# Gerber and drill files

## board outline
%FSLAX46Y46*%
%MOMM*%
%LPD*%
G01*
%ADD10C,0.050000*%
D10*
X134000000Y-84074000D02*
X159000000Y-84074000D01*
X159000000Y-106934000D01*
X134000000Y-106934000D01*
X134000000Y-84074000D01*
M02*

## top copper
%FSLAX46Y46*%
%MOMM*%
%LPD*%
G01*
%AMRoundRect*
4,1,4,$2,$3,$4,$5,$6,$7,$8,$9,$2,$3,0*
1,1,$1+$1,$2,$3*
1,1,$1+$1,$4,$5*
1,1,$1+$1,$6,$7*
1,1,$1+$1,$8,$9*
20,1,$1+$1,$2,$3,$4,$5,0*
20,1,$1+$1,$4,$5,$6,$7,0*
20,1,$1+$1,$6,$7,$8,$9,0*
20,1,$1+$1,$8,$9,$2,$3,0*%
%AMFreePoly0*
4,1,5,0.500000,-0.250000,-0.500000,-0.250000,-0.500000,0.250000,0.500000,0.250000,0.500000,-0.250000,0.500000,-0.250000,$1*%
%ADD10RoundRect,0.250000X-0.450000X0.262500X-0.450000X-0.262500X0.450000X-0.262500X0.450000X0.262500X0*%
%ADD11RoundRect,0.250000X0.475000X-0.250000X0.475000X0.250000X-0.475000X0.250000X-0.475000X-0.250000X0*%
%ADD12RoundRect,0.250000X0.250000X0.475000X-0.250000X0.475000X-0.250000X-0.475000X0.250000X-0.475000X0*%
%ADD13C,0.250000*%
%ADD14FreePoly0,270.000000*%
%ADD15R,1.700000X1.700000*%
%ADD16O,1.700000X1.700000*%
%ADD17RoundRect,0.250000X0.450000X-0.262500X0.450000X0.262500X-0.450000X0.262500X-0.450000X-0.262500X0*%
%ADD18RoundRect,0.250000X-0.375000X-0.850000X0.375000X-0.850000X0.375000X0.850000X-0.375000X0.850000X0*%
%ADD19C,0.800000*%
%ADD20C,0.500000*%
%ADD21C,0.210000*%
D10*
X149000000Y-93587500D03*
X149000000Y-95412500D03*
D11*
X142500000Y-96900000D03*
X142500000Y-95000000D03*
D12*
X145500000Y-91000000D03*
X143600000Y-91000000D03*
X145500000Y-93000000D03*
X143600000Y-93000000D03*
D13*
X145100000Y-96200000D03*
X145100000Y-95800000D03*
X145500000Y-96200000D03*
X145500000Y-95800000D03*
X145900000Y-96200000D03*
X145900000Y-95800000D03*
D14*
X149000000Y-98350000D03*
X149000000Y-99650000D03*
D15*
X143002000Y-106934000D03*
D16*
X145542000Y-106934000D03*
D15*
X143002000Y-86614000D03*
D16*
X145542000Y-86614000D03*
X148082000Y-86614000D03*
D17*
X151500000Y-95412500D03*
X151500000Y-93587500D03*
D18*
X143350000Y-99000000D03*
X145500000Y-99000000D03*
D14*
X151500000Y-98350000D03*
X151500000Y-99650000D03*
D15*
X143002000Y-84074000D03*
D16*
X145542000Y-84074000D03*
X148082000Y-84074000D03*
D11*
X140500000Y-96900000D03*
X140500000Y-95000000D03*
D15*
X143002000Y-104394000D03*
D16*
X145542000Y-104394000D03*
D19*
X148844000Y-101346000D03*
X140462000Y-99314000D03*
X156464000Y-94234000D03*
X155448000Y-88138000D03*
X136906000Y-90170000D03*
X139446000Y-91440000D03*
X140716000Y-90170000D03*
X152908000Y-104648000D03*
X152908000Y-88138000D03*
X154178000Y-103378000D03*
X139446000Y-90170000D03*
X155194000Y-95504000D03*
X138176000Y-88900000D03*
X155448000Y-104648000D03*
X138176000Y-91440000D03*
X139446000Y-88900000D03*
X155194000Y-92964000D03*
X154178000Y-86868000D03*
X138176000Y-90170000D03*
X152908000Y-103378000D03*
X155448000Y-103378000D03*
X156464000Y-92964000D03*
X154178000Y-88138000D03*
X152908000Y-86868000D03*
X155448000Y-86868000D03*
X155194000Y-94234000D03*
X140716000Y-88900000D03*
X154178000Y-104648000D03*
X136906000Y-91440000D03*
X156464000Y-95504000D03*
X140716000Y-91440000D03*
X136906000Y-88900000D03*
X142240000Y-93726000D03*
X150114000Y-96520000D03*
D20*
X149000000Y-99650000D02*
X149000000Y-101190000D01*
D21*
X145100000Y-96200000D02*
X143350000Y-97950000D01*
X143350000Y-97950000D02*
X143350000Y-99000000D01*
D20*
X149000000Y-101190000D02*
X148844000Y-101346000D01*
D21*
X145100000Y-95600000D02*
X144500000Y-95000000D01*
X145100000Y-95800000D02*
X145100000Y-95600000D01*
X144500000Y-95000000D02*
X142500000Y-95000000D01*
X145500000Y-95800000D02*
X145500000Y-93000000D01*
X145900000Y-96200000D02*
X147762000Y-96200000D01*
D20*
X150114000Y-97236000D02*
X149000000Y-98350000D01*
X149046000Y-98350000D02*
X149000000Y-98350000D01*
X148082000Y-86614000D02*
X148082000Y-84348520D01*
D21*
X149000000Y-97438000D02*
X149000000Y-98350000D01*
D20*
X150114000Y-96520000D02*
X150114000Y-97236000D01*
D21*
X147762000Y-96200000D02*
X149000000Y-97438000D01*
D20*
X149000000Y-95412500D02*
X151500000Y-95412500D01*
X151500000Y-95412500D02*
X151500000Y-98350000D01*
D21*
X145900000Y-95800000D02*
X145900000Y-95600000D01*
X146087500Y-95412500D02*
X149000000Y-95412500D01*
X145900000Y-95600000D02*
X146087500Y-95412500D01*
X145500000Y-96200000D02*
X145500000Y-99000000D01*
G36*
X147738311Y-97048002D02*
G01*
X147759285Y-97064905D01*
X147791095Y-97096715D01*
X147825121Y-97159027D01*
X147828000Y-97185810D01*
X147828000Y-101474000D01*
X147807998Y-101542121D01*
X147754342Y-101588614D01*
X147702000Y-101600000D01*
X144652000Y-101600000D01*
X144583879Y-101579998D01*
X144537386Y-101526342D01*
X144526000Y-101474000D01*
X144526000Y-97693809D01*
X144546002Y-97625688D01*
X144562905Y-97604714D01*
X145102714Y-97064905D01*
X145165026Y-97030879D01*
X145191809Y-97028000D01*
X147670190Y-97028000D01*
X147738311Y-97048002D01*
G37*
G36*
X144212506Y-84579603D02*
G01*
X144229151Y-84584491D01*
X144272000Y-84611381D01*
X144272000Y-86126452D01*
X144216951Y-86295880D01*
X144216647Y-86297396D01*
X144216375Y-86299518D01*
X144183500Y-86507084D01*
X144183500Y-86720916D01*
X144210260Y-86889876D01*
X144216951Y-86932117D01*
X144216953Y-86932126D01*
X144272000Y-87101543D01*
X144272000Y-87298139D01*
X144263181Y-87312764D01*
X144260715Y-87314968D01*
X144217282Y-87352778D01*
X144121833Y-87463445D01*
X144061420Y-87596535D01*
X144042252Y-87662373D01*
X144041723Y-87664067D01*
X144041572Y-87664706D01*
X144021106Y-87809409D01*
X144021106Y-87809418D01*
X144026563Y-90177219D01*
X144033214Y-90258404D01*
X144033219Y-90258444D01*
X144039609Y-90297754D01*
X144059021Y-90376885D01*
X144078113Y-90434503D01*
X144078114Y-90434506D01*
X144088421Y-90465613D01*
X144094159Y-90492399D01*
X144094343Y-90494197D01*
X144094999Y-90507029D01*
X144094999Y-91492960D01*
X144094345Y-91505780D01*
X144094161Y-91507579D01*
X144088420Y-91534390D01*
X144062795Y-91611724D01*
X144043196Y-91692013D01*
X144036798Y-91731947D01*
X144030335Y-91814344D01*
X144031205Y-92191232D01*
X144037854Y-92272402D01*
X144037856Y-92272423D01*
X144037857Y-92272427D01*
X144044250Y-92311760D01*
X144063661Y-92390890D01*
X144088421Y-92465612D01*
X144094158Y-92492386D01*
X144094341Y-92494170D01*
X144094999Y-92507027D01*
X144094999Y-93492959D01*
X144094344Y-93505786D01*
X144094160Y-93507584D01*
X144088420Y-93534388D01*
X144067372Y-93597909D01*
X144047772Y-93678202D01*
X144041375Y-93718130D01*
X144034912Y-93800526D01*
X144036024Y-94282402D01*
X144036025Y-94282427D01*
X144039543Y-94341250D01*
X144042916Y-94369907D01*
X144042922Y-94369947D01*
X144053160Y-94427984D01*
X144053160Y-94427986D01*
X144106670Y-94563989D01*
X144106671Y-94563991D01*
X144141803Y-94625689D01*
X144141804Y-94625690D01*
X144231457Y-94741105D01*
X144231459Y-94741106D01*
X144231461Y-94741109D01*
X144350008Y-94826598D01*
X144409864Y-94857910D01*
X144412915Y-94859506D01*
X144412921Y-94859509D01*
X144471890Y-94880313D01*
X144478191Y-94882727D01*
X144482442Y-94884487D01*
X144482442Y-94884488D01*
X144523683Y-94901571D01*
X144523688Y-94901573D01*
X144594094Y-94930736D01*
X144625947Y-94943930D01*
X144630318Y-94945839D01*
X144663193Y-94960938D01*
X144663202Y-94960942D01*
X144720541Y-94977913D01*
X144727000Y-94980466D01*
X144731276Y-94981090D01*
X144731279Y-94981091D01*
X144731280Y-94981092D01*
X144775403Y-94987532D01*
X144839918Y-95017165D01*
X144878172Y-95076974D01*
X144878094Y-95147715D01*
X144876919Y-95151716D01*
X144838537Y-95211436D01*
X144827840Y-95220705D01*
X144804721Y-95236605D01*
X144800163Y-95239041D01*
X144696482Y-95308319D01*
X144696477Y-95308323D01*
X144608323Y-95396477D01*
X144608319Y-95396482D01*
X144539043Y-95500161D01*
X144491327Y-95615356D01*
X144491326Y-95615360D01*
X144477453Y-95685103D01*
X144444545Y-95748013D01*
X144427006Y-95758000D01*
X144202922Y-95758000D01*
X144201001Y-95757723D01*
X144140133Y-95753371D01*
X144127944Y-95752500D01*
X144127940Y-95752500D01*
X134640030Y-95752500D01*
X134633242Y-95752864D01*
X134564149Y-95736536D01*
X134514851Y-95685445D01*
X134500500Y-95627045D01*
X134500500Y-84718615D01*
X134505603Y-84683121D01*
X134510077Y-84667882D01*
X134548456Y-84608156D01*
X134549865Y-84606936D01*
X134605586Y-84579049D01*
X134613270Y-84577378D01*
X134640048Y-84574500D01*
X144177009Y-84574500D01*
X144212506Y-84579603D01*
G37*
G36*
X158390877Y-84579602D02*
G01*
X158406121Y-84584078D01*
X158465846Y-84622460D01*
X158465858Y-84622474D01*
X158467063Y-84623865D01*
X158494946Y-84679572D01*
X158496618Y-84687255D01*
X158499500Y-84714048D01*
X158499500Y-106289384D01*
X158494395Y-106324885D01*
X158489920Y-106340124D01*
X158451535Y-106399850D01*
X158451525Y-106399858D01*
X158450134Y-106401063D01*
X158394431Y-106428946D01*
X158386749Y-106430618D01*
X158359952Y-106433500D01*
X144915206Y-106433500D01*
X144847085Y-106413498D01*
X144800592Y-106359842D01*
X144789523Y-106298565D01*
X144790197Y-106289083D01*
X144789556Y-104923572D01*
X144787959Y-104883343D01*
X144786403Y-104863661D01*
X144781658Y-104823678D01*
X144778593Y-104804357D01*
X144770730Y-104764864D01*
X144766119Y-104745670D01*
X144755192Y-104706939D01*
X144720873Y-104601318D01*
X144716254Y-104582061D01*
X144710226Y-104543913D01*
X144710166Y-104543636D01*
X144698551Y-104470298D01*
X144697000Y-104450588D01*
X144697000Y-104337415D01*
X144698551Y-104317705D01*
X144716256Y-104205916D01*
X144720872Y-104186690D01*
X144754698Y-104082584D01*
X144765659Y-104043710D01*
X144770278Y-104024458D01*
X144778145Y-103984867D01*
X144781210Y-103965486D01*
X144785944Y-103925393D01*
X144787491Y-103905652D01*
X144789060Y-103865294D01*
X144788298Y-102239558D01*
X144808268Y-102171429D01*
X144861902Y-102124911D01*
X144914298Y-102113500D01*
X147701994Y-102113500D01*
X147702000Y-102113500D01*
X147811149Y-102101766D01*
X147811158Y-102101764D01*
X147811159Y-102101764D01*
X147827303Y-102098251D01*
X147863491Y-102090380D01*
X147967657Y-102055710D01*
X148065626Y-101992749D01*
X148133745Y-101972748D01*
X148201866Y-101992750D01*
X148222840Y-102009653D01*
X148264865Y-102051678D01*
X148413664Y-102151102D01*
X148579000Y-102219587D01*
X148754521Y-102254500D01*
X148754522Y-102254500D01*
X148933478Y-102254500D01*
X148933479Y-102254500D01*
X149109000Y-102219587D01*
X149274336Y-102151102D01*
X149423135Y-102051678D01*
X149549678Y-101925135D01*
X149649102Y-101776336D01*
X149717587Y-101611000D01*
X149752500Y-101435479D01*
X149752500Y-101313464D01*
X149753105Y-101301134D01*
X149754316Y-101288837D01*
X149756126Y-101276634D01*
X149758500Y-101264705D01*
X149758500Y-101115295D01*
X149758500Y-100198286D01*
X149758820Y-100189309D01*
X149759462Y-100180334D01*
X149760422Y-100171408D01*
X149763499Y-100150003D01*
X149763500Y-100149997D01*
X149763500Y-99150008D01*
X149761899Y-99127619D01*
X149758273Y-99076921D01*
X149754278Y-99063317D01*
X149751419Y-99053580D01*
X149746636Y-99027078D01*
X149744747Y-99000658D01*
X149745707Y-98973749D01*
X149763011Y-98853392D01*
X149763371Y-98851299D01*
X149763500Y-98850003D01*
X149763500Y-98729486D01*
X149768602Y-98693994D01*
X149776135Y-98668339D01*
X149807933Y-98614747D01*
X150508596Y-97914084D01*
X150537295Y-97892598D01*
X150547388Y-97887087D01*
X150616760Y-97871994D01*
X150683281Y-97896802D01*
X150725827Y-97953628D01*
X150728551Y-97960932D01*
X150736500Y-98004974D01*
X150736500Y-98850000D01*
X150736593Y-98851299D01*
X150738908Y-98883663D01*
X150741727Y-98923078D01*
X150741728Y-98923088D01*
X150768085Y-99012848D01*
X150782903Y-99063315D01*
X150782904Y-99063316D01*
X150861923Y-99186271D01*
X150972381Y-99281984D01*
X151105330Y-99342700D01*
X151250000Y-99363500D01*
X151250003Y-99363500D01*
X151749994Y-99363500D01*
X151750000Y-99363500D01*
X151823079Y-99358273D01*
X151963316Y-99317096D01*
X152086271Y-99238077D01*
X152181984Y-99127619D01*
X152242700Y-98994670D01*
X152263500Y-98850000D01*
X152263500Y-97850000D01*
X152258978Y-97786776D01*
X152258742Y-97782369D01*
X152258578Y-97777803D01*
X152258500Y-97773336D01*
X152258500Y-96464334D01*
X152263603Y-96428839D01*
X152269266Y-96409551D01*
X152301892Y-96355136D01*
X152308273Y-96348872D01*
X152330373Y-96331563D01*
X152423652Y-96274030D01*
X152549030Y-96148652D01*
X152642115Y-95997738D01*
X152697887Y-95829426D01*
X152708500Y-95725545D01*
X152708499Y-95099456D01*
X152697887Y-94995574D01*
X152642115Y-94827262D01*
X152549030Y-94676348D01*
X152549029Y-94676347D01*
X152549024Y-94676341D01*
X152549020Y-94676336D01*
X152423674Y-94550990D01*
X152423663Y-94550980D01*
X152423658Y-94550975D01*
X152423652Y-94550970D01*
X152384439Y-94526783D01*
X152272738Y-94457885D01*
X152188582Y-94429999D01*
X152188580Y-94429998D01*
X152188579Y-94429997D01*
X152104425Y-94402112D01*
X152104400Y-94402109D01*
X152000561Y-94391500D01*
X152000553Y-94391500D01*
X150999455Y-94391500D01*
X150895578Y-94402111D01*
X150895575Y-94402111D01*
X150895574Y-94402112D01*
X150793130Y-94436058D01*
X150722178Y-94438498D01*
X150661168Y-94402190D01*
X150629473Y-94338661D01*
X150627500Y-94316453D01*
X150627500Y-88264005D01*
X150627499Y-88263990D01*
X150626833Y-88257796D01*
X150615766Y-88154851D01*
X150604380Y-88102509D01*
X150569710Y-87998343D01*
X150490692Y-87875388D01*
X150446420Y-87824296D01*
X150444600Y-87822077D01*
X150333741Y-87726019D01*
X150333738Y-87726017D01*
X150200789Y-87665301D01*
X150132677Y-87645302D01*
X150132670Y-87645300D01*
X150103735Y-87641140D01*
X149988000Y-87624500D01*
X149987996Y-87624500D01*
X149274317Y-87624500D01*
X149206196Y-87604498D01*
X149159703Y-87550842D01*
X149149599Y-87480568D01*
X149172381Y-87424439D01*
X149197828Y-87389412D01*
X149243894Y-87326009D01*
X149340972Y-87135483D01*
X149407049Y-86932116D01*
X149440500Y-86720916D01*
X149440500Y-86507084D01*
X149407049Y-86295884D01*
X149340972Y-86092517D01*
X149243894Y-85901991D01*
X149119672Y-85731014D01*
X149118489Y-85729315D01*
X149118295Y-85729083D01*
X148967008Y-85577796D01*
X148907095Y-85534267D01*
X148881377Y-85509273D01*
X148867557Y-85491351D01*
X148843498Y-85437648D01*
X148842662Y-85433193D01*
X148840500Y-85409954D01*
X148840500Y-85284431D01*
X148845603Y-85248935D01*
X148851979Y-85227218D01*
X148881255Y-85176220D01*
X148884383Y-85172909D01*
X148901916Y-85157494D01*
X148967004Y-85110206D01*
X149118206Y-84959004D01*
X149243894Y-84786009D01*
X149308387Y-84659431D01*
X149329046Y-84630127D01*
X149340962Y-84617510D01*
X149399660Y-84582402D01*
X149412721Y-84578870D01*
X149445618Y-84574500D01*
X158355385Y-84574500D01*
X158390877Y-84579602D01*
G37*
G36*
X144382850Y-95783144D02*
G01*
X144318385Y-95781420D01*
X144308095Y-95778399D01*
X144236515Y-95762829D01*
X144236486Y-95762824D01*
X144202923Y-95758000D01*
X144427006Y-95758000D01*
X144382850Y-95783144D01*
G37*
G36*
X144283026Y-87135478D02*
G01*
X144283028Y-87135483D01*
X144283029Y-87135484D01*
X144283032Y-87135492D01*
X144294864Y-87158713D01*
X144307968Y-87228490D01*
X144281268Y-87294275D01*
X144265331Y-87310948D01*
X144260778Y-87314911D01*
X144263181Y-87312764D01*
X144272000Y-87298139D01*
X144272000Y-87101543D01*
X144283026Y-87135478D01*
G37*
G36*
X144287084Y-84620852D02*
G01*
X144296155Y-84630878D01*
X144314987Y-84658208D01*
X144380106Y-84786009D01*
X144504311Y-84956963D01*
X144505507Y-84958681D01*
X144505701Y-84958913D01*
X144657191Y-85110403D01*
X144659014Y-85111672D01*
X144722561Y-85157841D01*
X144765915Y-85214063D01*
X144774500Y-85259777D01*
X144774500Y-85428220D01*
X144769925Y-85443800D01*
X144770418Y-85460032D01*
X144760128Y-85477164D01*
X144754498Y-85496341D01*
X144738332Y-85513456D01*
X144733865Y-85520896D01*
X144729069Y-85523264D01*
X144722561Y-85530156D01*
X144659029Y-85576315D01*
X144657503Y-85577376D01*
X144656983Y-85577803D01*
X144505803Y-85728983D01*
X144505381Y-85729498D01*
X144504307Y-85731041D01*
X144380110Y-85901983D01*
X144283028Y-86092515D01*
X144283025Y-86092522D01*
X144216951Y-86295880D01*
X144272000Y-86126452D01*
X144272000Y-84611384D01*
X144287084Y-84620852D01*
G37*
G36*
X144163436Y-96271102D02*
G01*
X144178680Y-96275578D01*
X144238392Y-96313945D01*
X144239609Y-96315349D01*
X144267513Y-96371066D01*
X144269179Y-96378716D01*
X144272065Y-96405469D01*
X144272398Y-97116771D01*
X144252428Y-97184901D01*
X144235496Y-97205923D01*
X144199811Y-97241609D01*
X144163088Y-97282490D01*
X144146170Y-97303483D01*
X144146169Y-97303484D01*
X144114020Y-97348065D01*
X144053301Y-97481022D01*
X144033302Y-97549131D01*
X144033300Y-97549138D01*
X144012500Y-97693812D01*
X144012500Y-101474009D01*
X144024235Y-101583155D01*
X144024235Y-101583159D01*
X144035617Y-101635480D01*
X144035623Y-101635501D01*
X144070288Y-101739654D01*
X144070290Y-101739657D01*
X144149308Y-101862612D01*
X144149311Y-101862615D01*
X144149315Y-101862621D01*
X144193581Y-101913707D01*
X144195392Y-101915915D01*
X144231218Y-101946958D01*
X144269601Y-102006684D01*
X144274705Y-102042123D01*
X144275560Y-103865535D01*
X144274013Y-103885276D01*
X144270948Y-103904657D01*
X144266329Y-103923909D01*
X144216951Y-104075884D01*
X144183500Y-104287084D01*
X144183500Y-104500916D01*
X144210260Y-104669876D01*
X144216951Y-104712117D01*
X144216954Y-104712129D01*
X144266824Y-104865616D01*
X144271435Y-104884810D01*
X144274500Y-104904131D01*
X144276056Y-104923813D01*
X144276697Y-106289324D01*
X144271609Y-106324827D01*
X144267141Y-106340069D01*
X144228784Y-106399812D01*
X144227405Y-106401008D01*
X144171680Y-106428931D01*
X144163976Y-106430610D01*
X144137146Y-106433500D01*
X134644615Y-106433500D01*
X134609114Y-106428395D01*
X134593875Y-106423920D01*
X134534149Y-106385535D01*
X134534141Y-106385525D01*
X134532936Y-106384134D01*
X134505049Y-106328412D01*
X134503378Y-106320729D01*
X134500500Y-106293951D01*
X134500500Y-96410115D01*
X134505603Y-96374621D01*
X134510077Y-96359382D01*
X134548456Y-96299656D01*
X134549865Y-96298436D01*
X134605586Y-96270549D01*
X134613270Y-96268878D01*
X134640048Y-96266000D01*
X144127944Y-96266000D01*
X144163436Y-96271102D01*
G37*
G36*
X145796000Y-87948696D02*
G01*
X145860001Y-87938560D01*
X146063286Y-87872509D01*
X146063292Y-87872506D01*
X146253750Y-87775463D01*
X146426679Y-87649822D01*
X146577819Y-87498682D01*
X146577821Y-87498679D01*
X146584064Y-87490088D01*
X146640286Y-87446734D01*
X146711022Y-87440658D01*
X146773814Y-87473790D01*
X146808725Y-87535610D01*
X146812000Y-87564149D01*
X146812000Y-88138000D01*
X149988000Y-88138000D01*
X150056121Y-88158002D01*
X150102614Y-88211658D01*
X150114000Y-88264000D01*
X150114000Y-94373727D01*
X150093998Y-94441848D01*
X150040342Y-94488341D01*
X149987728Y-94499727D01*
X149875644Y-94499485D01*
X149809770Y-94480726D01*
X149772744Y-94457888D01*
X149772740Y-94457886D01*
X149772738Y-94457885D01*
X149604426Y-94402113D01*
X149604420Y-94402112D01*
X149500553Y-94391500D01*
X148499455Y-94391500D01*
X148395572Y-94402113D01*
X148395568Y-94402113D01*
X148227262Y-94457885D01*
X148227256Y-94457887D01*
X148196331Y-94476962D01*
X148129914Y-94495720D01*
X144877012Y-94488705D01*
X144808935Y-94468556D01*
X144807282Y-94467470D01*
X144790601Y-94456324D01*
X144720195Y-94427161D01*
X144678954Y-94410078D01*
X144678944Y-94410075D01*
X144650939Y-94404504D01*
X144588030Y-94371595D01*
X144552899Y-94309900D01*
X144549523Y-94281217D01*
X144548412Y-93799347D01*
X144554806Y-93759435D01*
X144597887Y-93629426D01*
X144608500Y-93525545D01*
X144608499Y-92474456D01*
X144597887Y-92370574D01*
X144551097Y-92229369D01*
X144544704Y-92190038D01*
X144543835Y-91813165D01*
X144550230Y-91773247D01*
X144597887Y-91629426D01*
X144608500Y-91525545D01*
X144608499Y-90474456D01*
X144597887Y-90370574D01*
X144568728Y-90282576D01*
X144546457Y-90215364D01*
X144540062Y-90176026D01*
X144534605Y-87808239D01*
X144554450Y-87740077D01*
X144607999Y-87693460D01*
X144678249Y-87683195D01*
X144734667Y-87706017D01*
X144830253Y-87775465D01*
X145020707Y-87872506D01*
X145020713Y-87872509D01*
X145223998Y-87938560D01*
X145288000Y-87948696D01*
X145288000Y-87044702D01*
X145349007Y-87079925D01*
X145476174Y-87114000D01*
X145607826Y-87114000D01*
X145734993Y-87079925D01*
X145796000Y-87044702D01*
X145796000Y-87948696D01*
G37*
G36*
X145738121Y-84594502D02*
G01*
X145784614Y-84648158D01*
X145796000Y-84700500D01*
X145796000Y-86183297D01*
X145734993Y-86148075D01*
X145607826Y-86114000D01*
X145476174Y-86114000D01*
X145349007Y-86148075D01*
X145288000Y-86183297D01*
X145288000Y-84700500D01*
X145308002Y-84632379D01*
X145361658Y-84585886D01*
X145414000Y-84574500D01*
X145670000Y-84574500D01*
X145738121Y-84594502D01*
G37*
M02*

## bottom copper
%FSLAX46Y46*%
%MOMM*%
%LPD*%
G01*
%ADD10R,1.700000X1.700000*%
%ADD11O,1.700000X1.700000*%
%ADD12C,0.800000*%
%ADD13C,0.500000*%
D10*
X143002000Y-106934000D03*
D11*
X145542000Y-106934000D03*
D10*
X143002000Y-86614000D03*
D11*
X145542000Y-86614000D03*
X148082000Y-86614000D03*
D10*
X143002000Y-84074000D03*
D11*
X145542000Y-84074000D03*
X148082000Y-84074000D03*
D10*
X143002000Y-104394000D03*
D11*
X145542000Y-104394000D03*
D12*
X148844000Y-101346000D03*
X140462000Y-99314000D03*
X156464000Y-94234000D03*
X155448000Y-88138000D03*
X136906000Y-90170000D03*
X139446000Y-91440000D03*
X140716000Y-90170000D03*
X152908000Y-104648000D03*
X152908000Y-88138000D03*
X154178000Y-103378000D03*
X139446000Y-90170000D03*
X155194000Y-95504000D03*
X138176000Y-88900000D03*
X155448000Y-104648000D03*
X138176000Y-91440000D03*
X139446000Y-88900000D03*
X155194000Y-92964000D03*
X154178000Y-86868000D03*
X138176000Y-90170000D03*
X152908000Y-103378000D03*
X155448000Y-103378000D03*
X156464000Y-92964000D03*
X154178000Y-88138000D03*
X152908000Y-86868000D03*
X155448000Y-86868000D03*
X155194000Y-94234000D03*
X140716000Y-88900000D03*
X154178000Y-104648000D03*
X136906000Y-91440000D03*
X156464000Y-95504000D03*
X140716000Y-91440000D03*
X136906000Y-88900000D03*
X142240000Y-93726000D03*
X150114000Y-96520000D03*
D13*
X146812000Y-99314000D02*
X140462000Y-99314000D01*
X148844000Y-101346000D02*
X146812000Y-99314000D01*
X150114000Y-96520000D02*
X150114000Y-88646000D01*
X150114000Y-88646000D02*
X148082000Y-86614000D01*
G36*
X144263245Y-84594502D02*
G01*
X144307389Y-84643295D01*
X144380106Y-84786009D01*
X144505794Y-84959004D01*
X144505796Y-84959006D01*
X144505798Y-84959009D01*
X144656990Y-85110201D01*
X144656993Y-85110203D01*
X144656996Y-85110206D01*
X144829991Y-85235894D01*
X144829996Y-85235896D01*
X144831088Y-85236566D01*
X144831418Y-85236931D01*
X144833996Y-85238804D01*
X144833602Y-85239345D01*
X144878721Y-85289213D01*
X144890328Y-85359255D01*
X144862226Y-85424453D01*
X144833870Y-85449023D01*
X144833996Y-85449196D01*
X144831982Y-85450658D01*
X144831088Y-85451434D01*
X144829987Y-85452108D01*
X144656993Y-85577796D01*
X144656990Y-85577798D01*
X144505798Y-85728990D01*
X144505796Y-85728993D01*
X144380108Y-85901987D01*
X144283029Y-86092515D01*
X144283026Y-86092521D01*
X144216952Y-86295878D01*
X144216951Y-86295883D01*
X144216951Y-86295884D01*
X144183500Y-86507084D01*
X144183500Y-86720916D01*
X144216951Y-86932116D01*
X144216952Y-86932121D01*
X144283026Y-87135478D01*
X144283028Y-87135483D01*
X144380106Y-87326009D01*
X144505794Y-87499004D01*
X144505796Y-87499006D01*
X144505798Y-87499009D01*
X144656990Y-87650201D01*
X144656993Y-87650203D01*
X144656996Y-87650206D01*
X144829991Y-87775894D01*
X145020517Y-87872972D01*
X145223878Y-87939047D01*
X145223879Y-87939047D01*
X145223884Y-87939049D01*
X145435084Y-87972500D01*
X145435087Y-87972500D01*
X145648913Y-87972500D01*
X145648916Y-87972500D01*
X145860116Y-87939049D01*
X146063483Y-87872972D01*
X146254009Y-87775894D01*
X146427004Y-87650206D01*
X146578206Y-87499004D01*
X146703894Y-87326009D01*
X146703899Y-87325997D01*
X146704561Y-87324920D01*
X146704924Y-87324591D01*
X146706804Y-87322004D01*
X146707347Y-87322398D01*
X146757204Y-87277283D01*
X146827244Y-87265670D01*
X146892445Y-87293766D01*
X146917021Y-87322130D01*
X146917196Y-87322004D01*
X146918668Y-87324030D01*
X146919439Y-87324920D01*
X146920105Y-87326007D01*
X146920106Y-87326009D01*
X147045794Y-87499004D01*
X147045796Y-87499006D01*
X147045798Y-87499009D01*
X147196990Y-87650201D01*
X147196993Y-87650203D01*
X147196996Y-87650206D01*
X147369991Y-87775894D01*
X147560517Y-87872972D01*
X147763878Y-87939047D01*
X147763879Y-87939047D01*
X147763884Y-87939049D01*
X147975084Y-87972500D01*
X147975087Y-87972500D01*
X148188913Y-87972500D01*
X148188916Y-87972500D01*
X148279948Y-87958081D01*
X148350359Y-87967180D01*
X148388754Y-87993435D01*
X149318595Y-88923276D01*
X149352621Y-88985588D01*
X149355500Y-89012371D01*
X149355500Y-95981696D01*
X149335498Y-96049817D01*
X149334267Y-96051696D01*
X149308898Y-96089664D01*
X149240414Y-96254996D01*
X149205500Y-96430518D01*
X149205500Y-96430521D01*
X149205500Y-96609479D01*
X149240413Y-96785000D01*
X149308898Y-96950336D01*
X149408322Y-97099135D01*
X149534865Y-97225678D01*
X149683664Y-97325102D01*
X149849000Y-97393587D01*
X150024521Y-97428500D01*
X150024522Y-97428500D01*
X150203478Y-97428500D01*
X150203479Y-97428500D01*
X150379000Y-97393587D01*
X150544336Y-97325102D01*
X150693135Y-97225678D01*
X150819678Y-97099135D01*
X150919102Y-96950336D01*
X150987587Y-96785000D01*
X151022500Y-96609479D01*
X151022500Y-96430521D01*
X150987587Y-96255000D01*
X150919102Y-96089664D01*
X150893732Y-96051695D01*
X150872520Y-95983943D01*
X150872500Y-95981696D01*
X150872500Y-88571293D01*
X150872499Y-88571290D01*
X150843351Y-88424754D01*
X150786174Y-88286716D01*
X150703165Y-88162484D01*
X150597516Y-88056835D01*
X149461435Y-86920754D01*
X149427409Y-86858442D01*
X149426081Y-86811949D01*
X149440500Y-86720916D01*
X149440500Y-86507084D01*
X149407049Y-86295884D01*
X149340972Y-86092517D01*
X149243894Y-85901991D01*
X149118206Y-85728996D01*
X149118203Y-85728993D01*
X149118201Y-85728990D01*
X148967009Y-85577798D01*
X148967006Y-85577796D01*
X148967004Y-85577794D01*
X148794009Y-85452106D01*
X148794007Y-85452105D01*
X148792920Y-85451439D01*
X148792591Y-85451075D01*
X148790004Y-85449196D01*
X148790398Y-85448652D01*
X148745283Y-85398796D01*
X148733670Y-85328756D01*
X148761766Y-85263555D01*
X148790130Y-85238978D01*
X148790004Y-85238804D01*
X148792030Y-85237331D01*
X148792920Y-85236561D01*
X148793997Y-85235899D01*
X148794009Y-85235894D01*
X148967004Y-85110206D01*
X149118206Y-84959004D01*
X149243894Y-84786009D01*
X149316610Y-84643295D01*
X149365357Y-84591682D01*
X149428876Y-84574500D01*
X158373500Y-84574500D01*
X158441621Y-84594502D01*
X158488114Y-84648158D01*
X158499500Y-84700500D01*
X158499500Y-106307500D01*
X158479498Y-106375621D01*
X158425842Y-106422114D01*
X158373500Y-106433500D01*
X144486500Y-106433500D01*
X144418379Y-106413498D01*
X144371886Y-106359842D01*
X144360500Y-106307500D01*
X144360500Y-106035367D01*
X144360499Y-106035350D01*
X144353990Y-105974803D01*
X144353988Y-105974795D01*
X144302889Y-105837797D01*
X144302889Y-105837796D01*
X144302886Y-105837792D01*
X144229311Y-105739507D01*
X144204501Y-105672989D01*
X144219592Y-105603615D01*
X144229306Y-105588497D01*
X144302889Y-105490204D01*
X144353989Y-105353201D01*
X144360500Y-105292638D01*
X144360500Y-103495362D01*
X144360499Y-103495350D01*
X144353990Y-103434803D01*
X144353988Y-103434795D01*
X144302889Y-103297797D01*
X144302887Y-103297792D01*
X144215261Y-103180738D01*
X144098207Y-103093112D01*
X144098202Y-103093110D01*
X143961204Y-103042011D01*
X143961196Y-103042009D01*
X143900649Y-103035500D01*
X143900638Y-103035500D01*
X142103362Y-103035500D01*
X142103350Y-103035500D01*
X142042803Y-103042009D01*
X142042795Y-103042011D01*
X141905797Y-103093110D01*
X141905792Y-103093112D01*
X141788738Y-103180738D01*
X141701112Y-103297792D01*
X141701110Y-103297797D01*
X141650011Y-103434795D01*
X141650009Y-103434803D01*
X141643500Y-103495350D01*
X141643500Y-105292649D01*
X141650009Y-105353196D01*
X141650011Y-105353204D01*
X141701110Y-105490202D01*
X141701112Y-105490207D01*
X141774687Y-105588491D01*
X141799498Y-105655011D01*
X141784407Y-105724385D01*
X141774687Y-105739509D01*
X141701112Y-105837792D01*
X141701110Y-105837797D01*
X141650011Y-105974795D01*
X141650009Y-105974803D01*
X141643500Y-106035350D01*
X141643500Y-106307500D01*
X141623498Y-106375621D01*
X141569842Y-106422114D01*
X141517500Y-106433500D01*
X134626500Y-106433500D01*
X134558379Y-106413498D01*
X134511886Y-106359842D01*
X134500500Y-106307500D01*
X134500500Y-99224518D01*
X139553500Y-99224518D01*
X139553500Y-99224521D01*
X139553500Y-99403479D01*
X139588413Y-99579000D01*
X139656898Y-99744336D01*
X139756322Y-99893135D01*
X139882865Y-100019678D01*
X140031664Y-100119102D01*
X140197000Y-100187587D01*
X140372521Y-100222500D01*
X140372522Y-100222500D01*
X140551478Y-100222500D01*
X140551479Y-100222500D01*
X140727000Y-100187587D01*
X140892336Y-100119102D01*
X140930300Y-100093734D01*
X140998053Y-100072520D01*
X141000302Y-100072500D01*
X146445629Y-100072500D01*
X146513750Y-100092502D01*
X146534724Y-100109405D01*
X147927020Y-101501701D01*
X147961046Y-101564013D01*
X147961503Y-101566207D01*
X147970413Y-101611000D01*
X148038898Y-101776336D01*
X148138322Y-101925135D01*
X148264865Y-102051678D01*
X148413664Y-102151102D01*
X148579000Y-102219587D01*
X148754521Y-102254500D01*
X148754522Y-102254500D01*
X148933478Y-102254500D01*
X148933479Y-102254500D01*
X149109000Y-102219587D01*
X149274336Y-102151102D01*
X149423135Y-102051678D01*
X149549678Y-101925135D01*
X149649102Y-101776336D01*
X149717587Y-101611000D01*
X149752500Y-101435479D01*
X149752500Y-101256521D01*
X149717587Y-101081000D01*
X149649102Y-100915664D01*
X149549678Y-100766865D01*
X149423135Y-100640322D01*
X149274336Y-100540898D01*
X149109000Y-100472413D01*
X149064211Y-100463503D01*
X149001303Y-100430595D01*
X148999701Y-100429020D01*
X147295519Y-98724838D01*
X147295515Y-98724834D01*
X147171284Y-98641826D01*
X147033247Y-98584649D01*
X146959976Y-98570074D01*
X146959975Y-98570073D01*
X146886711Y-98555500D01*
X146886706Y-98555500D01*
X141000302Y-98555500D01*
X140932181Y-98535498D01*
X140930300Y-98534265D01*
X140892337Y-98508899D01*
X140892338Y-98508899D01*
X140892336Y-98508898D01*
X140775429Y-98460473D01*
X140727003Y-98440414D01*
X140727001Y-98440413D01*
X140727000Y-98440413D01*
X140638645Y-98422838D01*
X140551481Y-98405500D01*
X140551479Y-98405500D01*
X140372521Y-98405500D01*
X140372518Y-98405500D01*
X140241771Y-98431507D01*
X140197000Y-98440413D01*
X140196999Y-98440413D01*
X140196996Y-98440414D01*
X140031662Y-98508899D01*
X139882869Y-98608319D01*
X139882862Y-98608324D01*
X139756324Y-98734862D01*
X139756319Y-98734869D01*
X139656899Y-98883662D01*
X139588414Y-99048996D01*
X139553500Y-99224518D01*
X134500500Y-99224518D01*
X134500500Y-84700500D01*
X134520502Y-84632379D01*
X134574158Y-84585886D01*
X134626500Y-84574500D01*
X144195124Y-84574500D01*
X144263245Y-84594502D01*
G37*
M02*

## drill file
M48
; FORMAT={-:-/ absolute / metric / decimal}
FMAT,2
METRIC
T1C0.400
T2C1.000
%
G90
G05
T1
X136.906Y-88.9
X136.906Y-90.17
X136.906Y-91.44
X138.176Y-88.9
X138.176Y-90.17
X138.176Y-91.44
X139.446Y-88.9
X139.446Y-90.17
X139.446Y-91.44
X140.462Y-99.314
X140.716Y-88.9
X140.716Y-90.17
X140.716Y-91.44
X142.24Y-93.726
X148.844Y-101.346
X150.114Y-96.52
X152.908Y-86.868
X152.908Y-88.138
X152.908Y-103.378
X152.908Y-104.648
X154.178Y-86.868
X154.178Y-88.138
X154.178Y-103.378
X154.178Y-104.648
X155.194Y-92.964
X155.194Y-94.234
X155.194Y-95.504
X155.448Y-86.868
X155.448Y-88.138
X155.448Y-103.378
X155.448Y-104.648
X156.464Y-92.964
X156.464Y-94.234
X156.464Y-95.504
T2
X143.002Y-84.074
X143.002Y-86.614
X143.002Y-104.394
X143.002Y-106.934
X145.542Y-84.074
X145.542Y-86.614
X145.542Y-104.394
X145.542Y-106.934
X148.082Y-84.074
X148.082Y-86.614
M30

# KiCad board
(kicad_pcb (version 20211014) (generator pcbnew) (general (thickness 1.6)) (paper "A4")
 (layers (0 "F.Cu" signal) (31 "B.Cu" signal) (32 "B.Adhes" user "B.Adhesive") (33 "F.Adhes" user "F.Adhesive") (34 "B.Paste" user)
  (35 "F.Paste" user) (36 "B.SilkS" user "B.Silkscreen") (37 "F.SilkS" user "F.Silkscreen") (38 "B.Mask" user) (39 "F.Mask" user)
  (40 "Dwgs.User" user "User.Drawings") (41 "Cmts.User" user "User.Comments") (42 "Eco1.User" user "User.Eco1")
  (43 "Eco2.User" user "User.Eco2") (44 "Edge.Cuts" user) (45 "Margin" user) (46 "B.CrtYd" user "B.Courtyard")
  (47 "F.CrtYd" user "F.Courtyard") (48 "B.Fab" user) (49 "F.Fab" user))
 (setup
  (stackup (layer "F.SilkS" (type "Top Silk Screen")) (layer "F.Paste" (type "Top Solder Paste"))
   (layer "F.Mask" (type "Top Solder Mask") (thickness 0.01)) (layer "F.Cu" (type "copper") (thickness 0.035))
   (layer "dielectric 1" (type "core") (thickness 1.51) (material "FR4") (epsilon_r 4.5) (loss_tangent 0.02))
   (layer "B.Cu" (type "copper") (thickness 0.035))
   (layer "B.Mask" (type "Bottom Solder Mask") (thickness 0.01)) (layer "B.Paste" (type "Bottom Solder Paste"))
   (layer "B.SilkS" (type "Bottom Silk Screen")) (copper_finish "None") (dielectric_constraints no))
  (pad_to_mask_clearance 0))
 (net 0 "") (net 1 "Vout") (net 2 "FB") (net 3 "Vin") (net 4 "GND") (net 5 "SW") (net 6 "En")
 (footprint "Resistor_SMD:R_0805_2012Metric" (layer "F.Cu") (at 149 94.5 -90) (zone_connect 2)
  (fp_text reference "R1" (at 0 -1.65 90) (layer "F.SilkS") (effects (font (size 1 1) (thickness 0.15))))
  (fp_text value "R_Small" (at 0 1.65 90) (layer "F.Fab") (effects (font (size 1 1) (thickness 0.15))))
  (pad "1" smd roundrect (at -0.9125 0 270) (size 1.025 1.4) (layers "F.Cu" "F.Paste" "F.Mask") (roundrect_rratio 0.243902) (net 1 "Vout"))
  (pad "2" smd roundrect (at 0.9125 0 270) (size 1.025 1.4) (layers "F.Cu" "F.Paste" "F.Mask") (roundrect_rratio 0.243902) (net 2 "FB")))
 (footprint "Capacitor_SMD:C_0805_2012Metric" (layer "F.Cu") (at 142.5 95.95 90) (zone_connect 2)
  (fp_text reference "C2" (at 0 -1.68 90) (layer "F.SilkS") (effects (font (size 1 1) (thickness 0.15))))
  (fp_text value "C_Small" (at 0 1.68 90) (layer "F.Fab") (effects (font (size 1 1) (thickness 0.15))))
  (pad "1" smd roundrect (at -0.95 0 90) (size 1 1.45) (layers "F.Cu" "F.Paste" "F.Mask") (roundrect_rratio 0.25) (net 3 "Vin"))
  (pad "2" smd roundrect (at 0.95 0 90) (size 1 1.45) (layers "F.Cu" "F.Paste" "F.Mask") (roundrect_rratio 0.25) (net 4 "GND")))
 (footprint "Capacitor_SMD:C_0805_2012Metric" (layer "F.Cu") (at 144.55 91 180) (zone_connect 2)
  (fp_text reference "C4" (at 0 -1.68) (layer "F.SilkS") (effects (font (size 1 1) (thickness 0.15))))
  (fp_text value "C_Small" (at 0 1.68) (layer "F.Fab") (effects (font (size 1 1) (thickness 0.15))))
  (pad "1" smd roundrect (at -0.95 0 180) (size 1 1.45) (layers "F.Cu" "F.Paste" "F.Mask") (roundrect_rratio 0.25) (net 1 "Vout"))
  (pad "2" smd roundrect (at 0.95 0 180) (size 1 1.45) (layers "F.Cu" "F.Paste" "F.Mask") (roundrect_rratio 0.25) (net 4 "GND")))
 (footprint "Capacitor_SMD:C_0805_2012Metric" (layer "F.Cu") (at 144.55 93 180) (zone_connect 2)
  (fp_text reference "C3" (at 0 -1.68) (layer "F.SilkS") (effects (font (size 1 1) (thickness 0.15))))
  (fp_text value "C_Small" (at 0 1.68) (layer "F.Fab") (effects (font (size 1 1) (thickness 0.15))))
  (pad "1" smd roundrect (at -0.95 0 180) (size 1 1.45) (layers "F.Cu" "F.Paste" "F.Mask") (roundrect_rratio 0.25) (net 1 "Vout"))
  (pad "2" smd roundrect (at 0.95 0 180) (size 1 1.45) (layers "F.Cu" "F.Paste" "F.Mask") (roundrect_rratio 0.25) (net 4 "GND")))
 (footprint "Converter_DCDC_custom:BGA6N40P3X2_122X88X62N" (layer "F.Cu") (at 145.5 96 90)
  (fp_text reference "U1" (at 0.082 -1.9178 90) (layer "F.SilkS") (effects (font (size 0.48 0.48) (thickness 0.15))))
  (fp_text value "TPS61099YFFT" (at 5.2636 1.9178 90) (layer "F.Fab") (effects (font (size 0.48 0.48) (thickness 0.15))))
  (pad "A1" smd circle (at -0.2 -0.4 90) (size 0.25 0.25) (layers "F.Cu" "F.Paste" "F.Mask") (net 3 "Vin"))
  (pad "A2" smd circle (at 0.2 -0.4 90) (size 0.25 0.25) (layers "F.Cu" "F.Paste" "F.Mask") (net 4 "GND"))
  (pad "B1" smd circle (at -0.2 0 90) (size 0.25 0.25) (layers "F.Cu" "F.Paste" "F.Mask") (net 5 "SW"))
  (pad "B2" smd circle (at 0.2 0 90) (size 0.25 0.25) (layers "F.Cu" "F.Paste" "F.Mask") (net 1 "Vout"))
  (pad "C1" smd circle (at -0.2 0.4 90) (size 0.25 0.25) (layers "F.Cu" "F.Paste" "F.Mask") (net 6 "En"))
  (pad "C2" smd circle (at 0.2 0.4 90) (size 0.25 0.25) (layers "F.Cu" "F.Paste" "F.Mask") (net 2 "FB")))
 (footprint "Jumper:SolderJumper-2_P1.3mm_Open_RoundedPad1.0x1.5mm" (layer "F.Cu") (at 149 99 -90)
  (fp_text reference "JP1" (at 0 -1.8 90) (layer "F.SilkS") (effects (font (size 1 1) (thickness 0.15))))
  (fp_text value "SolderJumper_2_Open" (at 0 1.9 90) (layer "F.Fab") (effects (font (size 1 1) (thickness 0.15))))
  (pad "1" smd custom (at -0.65 0 270) (size 1 0.5) (layers "F.Cu" "F.Mask") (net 6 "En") (zone_connect 2)
   (options (clearance outline) (anchor rect)) (primitives))
  (pad "2" smd custom (at 0.65 0 270) (size 1 0.5) (layers "F.Cu" "F.Mask") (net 3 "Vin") (zone_connect 2)
   (options (clearance outline) (anchor rect)) (primitives)))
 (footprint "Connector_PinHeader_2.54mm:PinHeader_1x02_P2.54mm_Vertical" (layer "F.Cu") (at 143.002 106.934 90) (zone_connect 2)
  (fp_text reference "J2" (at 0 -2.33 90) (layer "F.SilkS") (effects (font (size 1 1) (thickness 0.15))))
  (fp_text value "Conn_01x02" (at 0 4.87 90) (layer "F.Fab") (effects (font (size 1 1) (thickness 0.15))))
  (pad "1" thru_hole rect (at 0 0 90) (size 1.7 1.7) (drill 1) (layers *.Cu *.Mask) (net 3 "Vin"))
  (pad "2" thru_hole oval (at 0 2.54 90) (size 1.7 1.7) (drill 1) (layers *.Cu *.Mask) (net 4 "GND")))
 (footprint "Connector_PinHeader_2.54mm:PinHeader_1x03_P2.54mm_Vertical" (layer "F.Cu") (at 143.002 86.614 90)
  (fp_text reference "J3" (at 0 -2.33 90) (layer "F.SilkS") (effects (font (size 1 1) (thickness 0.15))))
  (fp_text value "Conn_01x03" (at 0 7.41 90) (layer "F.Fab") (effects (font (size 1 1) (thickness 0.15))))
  (pad "1" thru_hole rect (at 0 0 90) (size 1.7 1.7) (drill 1) (layers *.Cu *.Mask) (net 4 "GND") (zone_connect 2))
  (pad "2" thru_hole oval (at 0 2.54 90) (size 1.7 1.7) (drill 1) (layers *.Cu *.Mask) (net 1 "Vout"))
  (pad "3" thru_hole oval (at 0 5.08 90) (size 1.7 1.7) (drill 1) (layers *.Cu *.Mask) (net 6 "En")))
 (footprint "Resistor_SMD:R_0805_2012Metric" (layer "F.Cu") (at 151.5 94.5 90) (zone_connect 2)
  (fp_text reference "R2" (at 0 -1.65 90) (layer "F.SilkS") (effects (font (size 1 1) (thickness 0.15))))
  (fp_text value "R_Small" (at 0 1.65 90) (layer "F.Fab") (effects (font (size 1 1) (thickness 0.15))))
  (pad "1" smd roundrect (at -0.9125 0 90) (size 1.025 1.4) (layers "F.Cu" "F.Paste" "F.Mask") (roundrect_rratio 0.243902) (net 2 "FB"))
  (pad "2" smd roundrect (at 0.9125 0 90) (size 1.025 1.4) (layers "F.Cu" "F.Paste" "F.Mask") (roundrect_rratio 0.243902) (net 4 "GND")))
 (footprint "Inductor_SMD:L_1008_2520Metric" (layer "F.Cu") (at 144.425 99) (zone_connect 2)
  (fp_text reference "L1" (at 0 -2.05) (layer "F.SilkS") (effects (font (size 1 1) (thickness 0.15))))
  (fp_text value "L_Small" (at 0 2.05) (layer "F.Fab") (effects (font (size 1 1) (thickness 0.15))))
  (pad "1" smd roundrect (at -1.075 0) (size 1.25 2.2) (layers "F.Cu" "F.Paste" "F.Mask") (roundrect_rratio 0.2) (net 3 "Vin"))
  (pad "2" smd roundrect (at 1.075 0) (size 1.25 2.2) (layers "F.Cu" "F.Paste" "F.Mask") (roundrect_rratio 0.2) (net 5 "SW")))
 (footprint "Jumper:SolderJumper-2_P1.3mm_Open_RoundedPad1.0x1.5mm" (layer "F.Cu") (at 151.5 99 -90)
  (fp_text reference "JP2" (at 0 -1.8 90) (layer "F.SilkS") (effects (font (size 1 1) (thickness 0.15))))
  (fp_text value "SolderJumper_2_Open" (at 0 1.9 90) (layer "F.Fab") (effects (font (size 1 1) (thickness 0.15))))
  (pad "1" smd custom (at -0.65 0 270) (size 1 0.5) (layers "F.Cu" "F.Mask") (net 2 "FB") (zone_connect 2)
   (options (clearance outline) (anchor rect)) (primitives))
  (pad "2" smd custom (at 0.65 0 270) (size 1 0.5) (layers "F.Cu" "F.Mask") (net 4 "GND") (zone_connect 2)
   (options (clearance outline) (anchor rect)) (primitives)))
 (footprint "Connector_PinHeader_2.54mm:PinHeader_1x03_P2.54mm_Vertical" (layer "F.Cu") (at 143.002 84.074 90)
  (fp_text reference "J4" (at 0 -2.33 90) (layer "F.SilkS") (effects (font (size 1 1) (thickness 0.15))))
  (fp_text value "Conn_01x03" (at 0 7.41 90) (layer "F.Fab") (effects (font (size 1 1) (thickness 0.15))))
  (pad "1" thru_hole rect (at 0 0 90) (size 1.7 1.7) (drill 1) (layers *.Cu *.Mask) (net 4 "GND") (zone_connect 2))
  (pad "2" thru_hole oval (at 0 2.54 90) (size 1.7 1.7) (drill 1) (layers *.Cu *.Mask) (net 1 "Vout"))
  (pad "3" thru_hole oval (at 0 5.08 90) (size 1.7 1.7) (drill 1) (layers *.Cu *.Mask) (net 6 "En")))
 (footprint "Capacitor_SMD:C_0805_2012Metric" (layer "F.Cu") (at 140.5 95.95 90) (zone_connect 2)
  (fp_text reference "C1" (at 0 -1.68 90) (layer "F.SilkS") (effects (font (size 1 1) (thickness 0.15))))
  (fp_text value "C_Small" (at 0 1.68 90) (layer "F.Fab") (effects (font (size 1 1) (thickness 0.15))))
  (pad "1" smd roundrect (at -0.95 0 90) (size 1 1.45) (layers "F.Cu" "F.Paste" "F.Mask") (roundrect_rratio 0.25) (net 3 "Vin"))
  (pad "2" smd roundrect (at 0.95 0 90) (size 1 1.45) (layers "F.Cu" "F.Paste" "F.Mask") (roundrect_rratio 0.25) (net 4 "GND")))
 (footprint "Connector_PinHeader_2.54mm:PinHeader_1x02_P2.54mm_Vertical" (layer "F.Cu") (at 143.002 104.394 90) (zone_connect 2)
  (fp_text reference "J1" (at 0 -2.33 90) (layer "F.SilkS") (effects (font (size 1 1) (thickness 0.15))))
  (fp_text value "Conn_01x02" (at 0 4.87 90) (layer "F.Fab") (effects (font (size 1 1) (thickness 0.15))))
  (pad "1" thru_hole rect (at 0 0 90) (size 1.7 1.7) (drill 1) (layers *.Cu *.Mask) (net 3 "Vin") (zone_connect 2))
  (pad "2" thru_hole oval (at 0 2.54 90) (size 1.7 1.7) (drill 1) (layers *.Cu *.Mask) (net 4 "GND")))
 (gr_rect (start 134 84.074) (end 159 106.934) (layer "Edge.Cuts") (width 0.05) (fill none))
 (segment (start 149 99.65) (end 149 101.19) (width 0.5) (layer "F.Cu") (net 3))
 (segment (start 145.1 96.2) (end 143.35 97.95) (width 0.21) (layer "F.Cu") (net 3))
 (segment (start 143.35 97.95) (end 143.35 99) (width 0.21) (layer "F.Cu") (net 3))
 (segment (start 149 101.19) (end 148.844 101.346) (width 0.5) (layer "F.Cu") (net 3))
 (via (at 148.844 101.346) (size 0.8) (drill 0.4) (layers "F.Cu" "B.Cu") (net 3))
 (via (at 140.462 99.314) (size 0.8) (drill 0.4) (layers "F.Cu" "B.Cu") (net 3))
 (segment (start 146.812 99.314) (end 140.462 99.314) (width 0.5) (layer "B.Cu") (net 3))
 (segment (start 148.844 101.346) (end 146.812 99.314) (width 0.5) (layer "B.Cu") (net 3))
 (segment (start 145.1 95.6) (end 144.5 95) (width 0.21) (layer "F.Cu") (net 4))
 (segment (start 145.1 95.8) (end 145.1 95.6) (width 0.21) (layer "F.Cu") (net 4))
 (segment (start 144.5 95) (end 142.5 95) (width 0.21) (layer "F.Cu") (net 4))
 (via (at 156.464 94.234) (size 0.8) (drill 0.4) (layers "F.Cu" "B.Cu") (free) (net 4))
 (via (at 155.448 88.138) (size 0.8) (drill 0.4) (layers "F.Cu" "B.Cu") (free) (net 4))
 (via (at 136.906 90.17) (size 0.8) (drill 0.4) (layers "F.Cu" "B.Cu") (free) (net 4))
 (via (at 139.446 91.44) (size 0.8) (drill 0.4) (layers "F.Cu" "B.Cu") (free) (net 4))
 (via (at 140.716 90.17) (size 0.8) (drill 0.4) (layers "F.Cu" "B.Cu") (free) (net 4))
 (via (at 152.908 104.648) (size 0.8) (drill 0.4) (layers "F.Cu" "B.Cu") (free) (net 4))
 (via (at 152.908 88.138) (size 0.8) (drill 0.4) (layers "F.Cu" "B.Cu") (free) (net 4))
 (via (at 154.178 103.378) (size 0.8) (drill 0.4) (layers "F.Cu" "B.Cu") (free) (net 4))
 (via (at 139.446 90.17) (size 0.8) (drill 0.4) (layers "F.Cu" "B.Cu") (free) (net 4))
 (via (at 155.194 95.504) (size 0.8) (drill 0.4) (layers "F.Cu" "B.Cu") (free) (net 4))
 (via (at 138.176 88.9) (size 0.8) (drill 0.4) (layers "F.Cu" "B.Cu") (free) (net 4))
 (via (at 155.448 104.648) (size 0.8) (drill 0.4) (layers "F.Cu" "B.Cu") (free) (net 4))
 (via (at 138.176 91.44) (size 0.8) (drill 0.4) (layers "F.Cu" "B.Cu") (free) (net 4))
 (via (at 139.446 88.9) (size 0.8) (drill 0.4) (layers "F.Cu" "B.Cu") (free) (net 4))
 (via (at 155.194 92.964) (size 0.8) (drill 0.4) (layers "F.Cu" "B.Cu") (free) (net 4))
 (via (at 154.178 86.868) (size 0.8) (drill 0.4) (layers "F.Cu" "B.Cu") (free) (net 4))
 (via (at 138.176 90.17) (size 0.8) (drill 0.4) (layers "F.Cu" "B.Cu") (free) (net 4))
 (via (at 152.908 103.378) (size 0.8) (drill 0.4) (layers "F.Cu" "B.Cu") (free) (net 4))
 (via (at 155.448 103.378) (size 0.8) (drill 0.4) (layers "F.Cu" "B.Cu") (free) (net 4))
 (via (at 156.464 92.964) (size 0.8) (drill 0.4) (layers "F.Cu" "B.Cu") (free) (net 4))
 (via (at 154.178 88.138) (size 0.8) (drill 0.4) (layers "F.Cu" "B.Cu") (free) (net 4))
 (via (at 152.908 86.868) (size 0.8) (drill 0.4) (layers "F.Cu" "B.Cu") (free) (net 4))
 (via (at 155.448 86.868) (size 0.8) (drill 0.4) (layers "F.Cu" "B.Cu") (free) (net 4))
 (via (at 155.194 94.234) (size 0.8) (drill 0.4) (layers "F.Cu" "B.Cu") (free) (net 4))
 (via (at 140.716 88.9) (size 0.8) (drill 0.4) (layers "F.Cu" "B.Cu") (free) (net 4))
 (via (at 154.178 104.648) (size 0.8) (drill 0.4) (layers "F.Cu" "B.Cu") (free) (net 4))
 (via (at 136.906 91.44) (size 0.8) (drill 0.4) (layers "F.Cu" "B.Cu") (free) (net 4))
 (via (at 156.464 95.504) (size 0.8) (drill 0.4) (layers "F.Cu" "B.Cu") (free) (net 4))
 (via (at 140.716 91.44) (size 0.8) (drill 0.4) (layers "F.Cu" "B.Cu") (free) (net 4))
 (via (at 136.906 88.9) (size 0.8) (drill 0.4) (layers "F.Cu" "B.Cu") (free) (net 4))
 (via (at 142.24 93.726) (size 0.8) (drill 0.4) (layers "F.Cu" "B.Cu") (free) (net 4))
 (segment (start 145.5 95.8) (end 145.5 93) (width 0.21) (layer "F.Cu") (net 1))
 (segment (start 145.9 96.2) (end 147.762 96.2) (width 0.21) (layer "F.Cu") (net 6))
 (segment (start 150.114 97.236) (end 149 98.35) (width 0.5) (layer "F.Cu") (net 6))
 (segment (start 149.046 98.35) (end 149 98.35) (width 0.5) (layer "F.Cu") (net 6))
 (segment (start 148.082 86.614) (end 148.082 84.34852) (width 0.5) (layer "F.Cu") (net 6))
 (segment (start 149 97.438) (end 149 98.35) (width 0.21) (layer "F.Cu") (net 6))
 (segment (start 150.114 96.52) (end 150.114 97.236) (width 0.5) (layer "F.Cu") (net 6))
 (segment (start 147.762 96.2) (end 149 97.438) (width 0.21) (layer "F.Cu") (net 6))
 (via (at 150.114 96.52) (size 0.8) (drill 0.4) (layers "F.Cu" "B.Cu") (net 6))
 (segment (start 150.114 96.52) (end 150.114 88.646) (width 0.5) (layer "B.Cu") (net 6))
 (segment (start 150.114 88.646) (end 148.082 86.614) (width 0.5) (layer "B.Cu") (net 6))
 (segment (start 149 95.4125) (end 151.5 95.4125) (width 0.5) (layer "F.Cu") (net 2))
 (segment (start 151.5 95.4125) (end 151.5 98.35) (width 0.5) (layer "F.Cu") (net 2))
 (segment (start 145.9 95.8) (end 145.9 95.6) (width 0.21) (layer "F.Cu") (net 2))
 (segment (start 146.0875 95.4125) (end 149 95.4125) (width 0.21) (layer "F.Cu") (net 2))
 (segment (start 145.9 95.6) (end 146.0875 95.4125) (width 0.21) (layer "F.Cu") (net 2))
 (segment (start 145.5 96.2) (end 145.5 99) (width 0.21) (layer "F.Cu") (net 5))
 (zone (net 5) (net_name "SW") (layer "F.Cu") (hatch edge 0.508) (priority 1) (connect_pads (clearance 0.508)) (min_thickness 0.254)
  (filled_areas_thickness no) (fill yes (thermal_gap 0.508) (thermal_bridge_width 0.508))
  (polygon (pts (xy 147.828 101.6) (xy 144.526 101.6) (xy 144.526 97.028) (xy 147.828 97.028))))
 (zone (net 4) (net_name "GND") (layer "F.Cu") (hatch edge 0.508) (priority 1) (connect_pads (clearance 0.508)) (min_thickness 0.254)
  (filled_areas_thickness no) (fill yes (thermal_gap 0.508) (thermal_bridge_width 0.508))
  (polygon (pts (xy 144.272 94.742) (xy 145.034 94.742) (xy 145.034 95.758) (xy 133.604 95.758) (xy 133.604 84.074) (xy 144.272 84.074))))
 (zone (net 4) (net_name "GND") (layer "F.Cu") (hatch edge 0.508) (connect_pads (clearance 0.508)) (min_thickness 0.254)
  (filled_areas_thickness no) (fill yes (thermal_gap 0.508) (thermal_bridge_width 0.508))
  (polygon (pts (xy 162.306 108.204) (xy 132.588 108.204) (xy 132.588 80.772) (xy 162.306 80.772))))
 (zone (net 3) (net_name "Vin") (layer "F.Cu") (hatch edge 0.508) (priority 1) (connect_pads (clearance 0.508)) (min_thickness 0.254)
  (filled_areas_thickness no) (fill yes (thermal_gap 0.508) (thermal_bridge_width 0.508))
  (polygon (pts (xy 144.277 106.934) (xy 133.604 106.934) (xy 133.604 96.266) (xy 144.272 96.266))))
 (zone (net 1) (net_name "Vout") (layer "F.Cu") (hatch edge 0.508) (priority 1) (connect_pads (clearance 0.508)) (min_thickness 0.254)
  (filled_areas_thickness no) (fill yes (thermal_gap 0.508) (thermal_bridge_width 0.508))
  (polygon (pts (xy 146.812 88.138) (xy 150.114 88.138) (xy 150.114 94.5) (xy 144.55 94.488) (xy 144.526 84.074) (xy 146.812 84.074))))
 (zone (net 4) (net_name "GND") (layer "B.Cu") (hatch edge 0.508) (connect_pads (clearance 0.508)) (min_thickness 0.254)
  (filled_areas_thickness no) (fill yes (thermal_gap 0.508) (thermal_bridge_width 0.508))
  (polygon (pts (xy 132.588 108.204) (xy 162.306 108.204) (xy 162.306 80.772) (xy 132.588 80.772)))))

